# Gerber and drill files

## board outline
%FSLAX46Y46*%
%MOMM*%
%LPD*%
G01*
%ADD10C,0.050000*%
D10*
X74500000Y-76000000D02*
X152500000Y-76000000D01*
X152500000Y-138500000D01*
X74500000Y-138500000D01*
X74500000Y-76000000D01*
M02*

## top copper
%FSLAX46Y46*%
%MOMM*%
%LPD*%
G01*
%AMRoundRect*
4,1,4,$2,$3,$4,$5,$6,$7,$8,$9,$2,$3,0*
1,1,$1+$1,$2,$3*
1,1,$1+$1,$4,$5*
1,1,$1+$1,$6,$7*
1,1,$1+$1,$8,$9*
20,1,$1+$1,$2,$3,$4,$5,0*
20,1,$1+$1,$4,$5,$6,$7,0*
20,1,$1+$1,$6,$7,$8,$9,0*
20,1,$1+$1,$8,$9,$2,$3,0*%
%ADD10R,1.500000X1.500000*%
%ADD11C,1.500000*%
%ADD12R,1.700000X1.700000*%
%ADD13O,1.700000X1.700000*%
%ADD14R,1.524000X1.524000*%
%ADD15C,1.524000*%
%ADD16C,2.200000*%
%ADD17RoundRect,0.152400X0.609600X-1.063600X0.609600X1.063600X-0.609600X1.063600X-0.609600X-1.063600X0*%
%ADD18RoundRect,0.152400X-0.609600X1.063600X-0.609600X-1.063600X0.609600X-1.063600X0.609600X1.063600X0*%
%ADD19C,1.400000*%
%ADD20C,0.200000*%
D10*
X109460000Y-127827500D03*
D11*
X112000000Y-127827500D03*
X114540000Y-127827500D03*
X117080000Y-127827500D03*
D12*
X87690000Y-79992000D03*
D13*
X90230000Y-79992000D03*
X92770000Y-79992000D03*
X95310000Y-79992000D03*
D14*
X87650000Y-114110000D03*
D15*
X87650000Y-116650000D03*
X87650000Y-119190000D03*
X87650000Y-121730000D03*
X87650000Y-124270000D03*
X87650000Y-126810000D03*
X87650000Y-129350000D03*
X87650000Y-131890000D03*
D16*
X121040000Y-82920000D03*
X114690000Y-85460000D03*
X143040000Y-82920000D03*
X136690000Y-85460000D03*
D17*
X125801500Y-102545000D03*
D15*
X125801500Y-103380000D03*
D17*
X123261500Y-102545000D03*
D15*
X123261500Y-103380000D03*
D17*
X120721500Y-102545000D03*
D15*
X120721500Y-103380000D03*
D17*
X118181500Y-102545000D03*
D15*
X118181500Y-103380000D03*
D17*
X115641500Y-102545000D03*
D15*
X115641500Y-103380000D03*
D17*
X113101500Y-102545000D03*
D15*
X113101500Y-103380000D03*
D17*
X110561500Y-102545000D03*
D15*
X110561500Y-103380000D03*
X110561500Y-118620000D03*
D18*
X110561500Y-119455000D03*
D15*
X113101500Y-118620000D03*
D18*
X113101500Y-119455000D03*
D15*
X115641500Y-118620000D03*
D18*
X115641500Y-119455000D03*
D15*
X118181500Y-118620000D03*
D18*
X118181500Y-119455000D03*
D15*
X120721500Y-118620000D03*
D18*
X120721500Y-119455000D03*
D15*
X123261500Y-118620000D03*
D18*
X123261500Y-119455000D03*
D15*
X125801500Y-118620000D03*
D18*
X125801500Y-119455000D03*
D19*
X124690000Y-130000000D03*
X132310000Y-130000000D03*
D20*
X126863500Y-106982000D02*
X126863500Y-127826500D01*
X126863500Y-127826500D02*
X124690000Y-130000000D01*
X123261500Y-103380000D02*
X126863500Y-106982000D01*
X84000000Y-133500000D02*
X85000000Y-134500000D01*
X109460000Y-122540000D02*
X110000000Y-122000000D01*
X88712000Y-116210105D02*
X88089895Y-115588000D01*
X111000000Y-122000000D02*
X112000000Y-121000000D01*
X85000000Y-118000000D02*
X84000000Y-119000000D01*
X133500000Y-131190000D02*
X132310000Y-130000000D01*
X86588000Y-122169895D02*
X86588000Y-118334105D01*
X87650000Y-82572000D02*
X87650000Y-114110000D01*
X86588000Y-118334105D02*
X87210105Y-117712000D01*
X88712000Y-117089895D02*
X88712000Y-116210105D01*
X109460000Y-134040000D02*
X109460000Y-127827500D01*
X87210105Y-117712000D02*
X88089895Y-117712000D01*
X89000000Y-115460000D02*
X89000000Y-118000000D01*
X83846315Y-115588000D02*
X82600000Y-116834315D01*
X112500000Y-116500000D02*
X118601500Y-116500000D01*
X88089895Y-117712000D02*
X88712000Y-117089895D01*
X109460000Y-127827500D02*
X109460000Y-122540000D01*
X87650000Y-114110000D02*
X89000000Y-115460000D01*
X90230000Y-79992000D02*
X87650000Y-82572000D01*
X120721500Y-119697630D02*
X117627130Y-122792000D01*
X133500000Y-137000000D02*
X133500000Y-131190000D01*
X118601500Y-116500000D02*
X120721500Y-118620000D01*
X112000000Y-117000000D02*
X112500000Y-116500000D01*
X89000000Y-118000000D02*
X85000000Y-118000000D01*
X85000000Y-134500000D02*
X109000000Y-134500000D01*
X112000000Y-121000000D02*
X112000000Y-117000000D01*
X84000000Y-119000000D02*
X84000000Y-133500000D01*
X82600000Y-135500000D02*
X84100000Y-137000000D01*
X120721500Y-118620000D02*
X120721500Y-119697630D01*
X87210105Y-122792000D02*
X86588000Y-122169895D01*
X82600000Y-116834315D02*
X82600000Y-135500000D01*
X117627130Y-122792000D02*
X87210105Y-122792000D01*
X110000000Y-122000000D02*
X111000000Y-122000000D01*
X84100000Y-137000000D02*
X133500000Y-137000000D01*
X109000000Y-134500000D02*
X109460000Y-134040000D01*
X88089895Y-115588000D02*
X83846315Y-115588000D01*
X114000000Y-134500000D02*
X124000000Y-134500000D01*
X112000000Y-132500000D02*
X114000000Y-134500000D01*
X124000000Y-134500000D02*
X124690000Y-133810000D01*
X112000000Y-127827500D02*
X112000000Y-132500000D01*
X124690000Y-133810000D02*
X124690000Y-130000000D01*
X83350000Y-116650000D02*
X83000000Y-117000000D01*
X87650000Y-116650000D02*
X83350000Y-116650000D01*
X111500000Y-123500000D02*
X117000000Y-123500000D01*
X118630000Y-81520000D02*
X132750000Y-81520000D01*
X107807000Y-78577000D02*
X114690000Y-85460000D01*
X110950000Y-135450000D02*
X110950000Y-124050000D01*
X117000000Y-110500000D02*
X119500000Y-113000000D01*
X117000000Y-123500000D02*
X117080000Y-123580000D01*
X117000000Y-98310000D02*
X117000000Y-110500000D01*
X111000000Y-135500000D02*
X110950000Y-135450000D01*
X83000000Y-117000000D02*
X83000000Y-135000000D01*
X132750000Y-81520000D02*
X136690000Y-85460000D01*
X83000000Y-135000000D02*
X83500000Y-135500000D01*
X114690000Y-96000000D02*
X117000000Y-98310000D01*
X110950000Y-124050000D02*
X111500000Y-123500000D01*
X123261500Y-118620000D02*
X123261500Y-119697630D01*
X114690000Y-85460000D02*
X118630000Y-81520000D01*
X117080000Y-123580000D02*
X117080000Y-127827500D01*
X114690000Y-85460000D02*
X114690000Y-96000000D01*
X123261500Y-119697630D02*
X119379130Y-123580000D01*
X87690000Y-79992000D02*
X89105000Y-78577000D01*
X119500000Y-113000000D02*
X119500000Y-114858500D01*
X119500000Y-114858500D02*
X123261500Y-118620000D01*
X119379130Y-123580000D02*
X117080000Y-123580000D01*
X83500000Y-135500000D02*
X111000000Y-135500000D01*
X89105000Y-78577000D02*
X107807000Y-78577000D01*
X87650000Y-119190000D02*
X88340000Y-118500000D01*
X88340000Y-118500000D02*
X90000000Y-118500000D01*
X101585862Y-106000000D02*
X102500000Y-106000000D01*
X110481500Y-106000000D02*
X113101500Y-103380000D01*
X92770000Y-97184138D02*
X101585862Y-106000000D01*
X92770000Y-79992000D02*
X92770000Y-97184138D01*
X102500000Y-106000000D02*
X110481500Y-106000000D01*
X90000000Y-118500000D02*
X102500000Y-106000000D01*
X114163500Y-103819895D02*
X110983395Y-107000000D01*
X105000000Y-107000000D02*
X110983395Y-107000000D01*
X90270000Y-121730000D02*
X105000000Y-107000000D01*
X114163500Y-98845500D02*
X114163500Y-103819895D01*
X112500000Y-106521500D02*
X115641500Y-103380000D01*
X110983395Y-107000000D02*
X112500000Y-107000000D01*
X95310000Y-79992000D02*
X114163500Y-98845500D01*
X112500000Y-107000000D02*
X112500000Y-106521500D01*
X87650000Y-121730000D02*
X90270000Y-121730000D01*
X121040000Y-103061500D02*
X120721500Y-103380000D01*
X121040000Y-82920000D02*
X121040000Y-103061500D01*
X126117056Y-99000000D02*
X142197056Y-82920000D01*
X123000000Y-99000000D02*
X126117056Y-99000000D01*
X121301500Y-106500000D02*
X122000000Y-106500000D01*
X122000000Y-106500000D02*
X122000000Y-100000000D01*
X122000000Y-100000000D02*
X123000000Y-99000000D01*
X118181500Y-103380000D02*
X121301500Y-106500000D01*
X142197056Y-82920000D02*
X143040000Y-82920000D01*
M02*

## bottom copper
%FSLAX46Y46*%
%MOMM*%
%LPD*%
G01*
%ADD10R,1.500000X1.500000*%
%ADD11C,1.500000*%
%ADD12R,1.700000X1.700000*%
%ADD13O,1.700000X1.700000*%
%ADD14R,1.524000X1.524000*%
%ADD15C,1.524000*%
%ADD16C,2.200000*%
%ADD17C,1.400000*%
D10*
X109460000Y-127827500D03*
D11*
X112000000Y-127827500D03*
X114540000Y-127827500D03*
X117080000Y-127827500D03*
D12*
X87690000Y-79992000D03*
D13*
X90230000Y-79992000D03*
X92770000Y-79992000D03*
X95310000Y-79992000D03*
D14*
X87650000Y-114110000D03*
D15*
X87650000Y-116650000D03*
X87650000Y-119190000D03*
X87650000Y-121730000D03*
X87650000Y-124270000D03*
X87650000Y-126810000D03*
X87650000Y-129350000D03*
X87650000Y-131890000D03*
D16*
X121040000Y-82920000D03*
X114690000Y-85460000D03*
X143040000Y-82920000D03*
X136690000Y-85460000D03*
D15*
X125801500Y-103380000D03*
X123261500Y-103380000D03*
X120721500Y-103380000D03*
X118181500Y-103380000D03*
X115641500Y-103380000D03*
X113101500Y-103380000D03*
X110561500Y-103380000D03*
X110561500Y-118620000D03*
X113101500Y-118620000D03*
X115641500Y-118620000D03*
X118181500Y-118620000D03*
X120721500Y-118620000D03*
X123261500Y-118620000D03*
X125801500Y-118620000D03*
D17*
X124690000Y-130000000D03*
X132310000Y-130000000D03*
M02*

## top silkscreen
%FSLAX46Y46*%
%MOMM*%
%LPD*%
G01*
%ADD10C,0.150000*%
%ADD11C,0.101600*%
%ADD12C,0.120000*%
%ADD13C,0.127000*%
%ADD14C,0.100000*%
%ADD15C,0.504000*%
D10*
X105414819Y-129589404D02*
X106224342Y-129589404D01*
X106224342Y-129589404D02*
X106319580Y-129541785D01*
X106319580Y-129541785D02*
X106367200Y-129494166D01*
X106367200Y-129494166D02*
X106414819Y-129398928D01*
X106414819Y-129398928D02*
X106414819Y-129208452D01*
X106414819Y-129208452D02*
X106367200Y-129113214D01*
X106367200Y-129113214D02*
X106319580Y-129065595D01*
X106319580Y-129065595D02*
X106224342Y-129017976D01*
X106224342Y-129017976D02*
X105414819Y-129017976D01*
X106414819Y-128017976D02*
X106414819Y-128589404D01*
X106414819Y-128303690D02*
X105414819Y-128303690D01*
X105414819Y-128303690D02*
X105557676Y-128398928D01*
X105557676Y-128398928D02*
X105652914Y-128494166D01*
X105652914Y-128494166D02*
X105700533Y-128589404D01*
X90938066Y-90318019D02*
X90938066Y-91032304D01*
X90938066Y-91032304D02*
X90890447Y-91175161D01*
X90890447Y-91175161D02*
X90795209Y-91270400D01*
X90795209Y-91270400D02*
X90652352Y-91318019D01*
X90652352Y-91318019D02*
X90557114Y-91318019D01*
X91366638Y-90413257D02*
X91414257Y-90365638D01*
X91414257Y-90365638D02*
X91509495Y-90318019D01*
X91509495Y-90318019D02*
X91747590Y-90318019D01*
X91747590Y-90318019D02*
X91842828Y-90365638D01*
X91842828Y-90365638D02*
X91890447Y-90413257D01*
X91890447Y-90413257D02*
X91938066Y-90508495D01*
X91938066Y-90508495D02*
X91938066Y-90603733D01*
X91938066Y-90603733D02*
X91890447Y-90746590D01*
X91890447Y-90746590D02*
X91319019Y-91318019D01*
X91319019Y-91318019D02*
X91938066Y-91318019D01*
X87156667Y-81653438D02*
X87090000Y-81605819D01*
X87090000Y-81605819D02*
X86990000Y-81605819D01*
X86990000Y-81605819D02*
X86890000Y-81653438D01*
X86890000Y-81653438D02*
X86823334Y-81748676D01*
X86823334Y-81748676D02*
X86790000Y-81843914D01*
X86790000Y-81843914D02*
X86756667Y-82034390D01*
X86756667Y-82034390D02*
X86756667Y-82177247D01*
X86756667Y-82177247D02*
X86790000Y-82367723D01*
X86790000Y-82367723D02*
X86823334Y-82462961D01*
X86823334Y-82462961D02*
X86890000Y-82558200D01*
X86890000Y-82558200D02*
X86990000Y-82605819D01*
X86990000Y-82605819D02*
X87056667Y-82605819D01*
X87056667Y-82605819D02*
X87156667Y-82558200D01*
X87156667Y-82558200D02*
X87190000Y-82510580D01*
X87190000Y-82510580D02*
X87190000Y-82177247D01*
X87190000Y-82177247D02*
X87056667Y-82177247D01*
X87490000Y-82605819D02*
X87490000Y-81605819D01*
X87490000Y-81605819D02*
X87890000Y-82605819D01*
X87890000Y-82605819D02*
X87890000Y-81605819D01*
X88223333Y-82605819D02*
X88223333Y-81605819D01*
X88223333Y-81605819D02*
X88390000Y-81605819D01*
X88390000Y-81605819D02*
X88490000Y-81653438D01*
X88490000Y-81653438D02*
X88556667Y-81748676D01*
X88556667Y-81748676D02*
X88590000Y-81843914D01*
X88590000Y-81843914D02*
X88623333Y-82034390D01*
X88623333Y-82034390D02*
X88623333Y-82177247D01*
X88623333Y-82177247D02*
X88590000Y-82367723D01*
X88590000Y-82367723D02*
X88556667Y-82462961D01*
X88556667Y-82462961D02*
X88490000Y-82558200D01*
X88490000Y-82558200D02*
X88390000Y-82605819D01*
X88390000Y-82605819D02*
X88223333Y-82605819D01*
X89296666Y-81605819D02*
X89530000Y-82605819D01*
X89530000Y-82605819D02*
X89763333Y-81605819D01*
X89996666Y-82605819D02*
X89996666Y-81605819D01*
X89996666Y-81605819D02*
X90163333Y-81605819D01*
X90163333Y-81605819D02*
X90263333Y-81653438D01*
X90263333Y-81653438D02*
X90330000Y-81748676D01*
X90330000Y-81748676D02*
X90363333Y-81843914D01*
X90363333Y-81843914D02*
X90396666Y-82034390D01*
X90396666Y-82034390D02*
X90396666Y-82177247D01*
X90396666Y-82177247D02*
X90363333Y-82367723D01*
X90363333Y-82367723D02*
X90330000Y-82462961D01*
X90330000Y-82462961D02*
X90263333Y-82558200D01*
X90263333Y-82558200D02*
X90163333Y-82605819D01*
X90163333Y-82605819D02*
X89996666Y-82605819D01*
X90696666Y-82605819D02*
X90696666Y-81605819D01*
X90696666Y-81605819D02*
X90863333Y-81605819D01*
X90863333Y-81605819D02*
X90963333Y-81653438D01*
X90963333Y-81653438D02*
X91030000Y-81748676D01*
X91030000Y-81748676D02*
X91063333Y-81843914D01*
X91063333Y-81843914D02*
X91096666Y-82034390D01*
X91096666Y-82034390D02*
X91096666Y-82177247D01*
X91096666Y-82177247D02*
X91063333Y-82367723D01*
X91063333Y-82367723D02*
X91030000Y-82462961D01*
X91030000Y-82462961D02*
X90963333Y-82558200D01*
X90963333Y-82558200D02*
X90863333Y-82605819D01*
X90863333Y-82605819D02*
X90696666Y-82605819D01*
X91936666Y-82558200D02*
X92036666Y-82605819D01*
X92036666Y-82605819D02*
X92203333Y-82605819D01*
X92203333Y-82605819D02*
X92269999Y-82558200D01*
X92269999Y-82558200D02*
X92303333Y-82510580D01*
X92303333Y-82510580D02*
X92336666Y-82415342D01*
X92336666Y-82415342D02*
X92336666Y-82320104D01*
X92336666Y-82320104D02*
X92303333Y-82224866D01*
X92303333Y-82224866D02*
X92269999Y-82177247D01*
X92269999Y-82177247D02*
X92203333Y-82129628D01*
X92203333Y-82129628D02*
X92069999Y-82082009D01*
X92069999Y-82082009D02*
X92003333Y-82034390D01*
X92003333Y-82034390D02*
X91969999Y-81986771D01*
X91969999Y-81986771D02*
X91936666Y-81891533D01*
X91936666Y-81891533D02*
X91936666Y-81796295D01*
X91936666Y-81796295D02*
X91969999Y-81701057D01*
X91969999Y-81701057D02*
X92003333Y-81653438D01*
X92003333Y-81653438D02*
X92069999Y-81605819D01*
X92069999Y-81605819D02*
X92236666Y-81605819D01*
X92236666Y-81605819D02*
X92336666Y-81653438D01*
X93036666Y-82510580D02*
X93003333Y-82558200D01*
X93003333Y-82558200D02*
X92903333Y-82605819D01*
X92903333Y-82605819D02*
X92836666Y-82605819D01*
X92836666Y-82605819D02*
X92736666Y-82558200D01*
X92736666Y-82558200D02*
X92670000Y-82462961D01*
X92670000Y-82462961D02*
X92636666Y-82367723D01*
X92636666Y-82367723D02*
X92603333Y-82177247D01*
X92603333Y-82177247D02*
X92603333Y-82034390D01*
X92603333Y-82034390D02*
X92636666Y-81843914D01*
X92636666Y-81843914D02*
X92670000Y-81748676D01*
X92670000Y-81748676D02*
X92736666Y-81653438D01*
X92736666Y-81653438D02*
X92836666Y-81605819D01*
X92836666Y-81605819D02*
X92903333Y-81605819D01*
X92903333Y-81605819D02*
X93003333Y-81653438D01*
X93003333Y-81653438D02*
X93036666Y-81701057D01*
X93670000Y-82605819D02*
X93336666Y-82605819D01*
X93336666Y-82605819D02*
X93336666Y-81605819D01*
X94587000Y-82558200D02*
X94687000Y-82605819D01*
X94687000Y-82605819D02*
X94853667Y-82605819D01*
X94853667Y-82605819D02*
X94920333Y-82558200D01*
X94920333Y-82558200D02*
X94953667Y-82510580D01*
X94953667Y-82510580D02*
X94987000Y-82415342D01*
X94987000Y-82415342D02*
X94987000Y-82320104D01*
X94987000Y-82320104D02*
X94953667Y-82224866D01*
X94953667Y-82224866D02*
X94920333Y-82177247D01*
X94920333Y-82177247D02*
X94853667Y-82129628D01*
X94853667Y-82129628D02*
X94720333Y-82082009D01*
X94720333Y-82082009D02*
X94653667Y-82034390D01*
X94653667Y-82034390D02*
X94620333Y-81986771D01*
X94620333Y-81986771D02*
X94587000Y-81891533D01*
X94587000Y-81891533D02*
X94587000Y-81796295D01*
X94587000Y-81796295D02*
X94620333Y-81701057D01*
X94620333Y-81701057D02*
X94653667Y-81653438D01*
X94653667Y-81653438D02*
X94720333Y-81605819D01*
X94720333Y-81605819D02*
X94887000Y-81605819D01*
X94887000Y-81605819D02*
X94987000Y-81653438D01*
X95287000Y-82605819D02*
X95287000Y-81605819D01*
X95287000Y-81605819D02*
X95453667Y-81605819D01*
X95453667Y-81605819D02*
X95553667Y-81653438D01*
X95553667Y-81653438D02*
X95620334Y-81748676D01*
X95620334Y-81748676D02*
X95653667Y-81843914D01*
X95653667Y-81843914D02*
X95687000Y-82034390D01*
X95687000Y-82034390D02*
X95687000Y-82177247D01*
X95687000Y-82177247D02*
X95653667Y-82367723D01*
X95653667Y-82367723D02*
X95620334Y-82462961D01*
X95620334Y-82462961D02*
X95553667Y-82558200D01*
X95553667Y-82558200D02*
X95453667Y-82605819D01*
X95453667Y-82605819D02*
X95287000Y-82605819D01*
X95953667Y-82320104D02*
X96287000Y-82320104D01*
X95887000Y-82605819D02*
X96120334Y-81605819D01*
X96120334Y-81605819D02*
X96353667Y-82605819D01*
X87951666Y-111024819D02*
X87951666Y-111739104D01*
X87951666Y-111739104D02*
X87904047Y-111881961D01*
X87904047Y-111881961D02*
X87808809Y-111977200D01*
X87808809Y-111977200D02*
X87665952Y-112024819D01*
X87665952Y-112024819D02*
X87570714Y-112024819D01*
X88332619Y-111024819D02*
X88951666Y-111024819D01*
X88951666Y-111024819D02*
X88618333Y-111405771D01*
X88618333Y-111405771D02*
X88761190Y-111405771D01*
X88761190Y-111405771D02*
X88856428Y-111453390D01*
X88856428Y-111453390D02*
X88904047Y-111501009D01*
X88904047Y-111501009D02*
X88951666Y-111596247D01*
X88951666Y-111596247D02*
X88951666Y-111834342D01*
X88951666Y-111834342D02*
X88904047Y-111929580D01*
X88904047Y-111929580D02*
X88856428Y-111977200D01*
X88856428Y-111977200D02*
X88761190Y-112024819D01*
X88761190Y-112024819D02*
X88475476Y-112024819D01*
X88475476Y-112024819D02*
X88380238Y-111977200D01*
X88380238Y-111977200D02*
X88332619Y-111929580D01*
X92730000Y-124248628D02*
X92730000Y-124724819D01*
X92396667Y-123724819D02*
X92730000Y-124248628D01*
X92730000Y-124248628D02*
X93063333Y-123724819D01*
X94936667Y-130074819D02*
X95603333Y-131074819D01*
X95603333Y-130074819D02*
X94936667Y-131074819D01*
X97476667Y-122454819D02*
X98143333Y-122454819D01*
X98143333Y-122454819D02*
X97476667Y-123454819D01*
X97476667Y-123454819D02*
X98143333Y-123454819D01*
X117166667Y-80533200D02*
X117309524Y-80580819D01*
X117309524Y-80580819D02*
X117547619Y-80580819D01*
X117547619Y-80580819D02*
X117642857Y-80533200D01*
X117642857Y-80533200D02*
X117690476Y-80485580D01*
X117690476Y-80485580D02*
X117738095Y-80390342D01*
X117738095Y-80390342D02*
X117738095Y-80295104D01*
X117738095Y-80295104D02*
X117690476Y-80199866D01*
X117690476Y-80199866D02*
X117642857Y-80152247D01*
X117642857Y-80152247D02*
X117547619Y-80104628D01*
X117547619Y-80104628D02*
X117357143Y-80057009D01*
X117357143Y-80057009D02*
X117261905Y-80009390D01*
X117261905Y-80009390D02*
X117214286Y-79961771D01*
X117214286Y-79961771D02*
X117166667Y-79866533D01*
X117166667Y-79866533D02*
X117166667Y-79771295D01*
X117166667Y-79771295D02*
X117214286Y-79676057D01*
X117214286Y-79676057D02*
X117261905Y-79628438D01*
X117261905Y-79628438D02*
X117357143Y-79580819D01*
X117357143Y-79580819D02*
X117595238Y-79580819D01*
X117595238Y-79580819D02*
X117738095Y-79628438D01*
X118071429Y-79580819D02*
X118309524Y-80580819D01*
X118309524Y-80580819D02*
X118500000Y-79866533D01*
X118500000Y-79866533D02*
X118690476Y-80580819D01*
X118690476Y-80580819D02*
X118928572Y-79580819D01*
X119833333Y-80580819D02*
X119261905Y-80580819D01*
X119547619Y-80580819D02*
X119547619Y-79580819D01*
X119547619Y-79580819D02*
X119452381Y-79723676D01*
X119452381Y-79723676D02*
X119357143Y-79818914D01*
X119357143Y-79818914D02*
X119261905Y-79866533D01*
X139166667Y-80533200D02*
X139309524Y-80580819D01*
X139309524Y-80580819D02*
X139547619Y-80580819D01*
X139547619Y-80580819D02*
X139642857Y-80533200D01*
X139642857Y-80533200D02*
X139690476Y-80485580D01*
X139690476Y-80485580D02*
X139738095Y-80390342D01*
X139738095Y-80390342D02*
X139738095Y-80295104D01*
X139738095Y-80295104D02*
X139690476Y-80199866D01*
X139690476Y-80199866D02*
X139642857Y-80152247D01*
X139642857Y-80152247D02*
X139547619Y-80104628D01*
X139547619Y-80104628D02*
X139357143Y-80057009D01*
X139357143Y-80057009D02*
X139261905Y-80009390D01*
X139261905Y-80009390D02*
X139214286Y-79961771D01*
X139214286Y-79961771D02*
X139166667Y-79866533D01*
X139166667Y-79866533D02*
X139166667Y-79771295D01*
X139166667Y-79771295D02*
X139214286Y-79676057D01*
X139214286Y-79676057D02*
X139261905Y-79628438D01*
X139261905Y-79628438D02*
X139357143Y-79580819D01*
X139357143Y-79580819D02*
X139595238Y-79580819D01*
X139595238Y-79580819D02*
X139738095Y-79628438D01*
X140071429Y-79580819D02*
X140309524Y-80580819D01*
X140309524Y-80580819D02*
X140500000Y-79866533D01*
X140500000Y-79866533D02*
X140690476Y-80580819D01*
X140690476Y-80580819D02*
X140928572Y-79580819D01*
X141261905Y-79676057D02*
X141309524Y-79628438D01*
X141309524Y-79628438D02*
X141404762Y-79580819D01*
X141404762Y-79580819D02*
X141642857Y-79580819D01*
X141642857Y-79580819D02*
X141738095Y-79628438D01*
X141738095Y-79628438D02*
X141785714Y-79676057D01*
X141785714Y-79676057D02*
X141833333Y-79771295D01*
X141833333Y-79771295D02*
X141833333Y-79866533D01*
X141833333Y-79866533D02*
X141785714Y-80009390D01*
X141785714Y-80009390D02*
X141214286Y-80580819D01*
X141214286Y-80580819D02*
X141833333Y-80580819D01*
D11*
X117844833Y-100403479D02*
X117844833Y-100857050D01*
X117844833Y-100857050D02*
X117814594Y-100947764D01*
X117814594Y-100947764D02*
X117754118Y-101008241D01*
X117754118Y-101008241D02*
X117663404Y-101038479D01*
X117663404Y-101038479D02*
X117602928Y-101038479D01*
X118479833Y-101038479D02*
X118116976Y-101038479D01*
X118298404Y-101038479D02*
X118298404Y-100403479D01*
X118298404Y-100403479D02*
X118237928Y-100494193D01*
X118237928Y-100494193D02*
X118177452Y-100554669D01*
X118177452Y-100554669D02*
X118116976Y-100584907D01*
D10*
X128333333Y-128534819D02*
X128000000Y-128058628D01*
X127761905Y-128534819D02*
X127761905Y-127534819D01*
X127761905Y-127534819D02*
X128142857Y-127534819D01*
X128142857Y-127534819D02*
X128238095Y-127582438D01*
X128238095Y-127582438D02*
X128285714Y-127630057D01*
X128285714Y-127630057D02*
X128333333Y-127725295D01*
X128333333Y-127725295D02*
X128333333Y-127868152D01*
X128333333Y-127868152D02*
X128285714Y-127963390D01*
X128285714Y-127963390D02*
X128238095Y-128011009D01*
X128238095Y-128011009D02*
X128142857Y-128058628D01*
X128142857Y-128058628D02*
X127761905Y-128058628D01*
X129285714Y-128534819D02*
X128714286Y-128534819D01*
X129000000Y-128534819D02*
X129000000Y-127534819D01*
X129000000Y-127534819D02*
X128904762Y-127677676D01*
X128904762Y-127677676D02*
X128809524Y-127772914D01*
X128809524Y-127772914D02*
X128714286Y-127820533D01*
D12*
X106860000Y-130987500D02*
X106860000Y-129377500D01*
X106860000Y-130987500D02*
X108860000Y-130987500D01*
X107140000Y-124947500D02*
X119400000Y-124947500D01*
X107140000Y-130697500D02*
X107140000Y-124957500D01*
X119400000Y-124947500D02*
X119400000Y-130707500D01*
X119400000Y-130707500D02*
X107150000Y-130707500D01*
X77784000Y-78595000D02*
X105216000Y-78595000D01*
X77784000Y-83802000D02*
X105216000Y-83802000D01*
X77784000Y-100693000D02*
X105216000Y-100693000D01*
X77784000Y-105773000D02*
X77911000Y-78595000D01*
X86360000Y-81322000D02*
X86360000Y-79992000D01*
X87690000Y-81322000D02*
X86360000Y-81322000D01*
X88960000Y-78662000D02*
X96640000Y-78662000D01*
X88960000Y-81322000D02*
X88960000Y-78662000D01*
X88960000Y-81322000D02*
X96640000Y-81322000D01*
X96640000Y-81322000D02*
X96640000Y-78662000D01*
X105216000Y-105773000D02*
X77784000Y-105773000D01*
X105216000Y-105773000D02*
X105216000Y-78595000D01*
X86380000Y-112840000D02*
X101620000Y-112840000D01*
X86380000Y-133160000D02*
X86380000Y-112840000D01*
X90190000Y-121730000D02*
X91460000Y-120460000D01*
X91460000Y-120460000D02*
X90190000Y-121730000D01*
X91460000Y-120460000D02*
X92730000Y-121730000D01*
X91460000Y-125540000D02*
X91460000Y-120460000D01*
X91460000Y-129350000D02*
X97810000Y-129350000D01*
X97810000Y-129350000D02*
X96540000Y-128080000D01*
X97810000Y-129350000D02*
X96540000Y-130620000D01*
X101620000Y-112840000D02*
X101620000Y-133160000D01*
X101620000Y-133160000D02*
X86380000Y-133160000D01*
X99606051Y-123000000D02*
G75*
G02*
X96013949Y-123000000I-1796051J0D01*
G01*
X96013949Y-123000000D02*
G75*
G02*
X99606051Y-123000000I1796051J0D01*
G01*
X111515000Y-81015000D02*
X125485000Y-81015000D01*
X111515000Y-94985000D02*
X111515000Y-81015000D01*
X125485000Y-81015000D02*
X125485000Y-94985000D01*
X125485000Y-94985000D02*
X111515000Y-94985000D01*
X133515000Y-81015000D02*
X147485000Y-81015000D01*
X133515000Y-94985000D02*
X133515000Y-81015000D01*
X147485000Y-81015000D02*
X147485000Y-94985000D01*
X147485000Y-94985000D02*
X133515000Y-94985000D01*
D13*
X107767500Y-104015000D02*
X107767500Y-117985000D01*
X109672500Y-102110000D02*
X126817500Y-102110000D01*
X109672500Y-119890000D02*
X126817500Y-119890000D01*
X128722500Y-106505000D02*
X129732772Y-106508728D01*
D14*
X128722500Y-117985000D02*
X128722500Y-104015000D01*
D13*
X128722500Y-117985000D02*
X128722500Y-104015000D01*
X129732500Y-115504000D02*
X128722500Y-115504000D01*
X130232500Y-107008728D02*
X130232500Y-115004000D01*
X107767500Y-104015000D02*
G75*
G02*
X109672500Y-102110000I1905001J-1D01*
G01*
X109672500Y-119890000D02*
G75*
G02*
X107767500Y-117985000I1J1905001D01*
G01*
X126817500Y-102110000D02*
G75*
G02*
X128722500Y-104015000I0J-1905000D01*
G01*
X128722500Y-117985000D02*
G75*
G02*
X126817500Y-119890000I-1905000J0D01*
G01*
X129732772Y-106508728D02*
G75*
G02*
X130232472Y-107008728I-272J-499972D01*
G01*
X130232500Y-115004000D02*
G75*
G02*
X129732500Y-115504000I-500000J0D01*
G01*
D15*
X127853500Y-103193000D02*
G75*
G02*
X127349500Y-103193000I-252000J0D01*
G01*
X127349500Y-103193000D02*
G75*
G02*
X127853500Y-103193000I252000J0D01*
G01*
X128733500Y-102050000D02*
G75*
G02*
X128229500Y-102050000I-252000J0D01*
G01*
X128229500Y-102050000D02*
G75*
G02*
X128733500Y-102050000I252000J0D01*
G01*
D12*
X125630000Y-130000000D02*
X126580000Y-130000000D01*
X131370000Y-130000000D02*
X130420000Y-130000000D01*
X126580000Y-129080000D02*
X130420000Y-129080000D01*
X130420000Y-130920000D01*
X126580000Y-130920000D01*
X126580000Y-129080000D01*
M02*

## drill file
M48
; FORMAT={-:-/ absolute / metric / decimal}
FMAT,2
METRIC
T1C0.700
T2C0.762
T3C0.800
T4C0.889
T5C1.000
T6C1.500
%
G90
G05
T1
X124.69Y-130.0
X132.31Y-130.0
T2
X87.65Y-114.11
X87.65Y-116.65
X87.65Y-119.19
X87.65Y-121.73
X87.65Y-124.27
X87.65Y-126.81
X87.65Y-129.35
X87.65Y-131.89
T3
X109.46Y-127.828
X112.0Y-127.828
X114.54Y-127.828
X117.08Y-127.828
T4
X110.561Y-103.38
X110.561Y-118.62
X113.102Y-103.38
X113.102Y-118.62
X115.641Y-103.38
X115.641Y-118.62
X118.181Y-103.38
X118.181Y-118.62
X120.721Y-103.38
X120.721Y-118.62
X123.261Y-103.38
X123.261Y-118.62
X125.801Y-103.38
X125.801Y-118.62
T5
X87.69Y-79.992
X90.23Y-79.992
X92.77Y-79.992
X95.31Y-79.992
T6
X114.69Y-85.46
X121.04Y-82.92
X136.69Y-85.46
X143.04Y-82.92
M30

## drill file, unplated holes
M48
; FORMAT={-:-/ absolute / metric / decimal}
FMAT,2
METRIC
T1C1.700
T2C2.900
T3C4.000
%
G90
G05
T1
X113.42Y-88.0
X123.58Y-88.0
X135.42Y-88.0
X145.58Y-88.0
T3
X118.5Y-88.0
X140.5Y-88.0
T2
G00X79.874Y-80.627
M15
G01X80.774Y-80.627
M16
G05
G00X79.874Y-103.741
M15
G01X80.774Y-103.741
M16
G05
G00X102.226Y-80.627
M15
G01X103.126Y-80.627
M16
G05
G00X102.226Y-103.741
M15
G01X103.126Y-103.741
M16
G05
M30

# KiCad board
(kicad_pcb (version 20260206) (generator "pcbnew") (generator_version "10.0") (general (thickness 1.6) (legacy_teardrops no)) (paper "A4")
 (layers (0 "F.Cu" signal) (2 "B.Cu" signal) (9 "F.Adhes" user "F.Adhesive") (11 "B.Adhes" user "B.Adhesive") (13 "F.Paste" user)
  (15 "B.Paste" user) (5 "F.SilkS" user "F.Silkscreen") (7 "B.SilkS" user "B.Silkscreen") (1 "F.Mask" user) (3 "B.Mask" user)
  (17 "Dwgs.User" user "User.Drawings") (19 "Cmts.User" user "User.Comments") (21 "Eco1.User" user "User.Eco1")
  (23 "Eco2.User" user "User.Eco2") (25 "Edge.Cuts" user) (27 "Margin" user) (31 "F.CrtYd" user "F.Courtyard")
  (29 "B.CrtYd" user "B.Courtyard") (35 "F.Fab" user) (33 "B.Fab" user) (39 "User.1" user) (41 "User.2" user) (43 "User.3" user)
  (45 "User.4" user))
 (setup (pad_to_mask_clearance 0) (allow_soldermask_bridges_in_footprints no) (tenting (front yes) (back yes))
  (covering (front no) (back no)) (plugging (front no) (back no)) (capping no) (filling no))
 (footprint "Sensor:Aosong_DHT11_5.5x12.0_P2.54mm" (layer "F.Cu") (at 109.46 127.8275 90)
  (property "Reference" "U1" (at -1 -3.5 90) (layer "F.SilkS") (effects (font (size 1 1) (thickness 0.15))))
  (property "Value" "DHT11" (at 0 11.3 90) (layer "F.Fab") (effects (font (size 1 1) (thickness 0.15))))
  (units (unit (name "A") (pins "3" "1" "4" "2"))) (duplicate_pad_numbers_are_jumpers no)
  (fp_line (start -3.16 -2.6) (end -1.55 -2.6) (stroke (width 0.12) (type solid)) (layer "F.SilkS"))
  (fp_line (start -3.16 -2.6) (end -3.16 -0.6) (stroke (width 0.12) (type solid)) (layer "F.SilkS"))
  (fp_line (start 2.88 -2.32) (end 2.88 9.94) (stroke (width 0.12) (type solid)) (layer "F.SilkS"))
  (fp_line (start -2.87 -2.32) (end 2.87 -2.32) (stroke (width 0.12) (type solid)) (layer "F.SilkS"))
  (fp_line (start 2.88 9.94) (end -2.88 9.94) (stroke (width 0.12) (type solid)) (layer "F.SilkS"))
  (fp_line (start -2.88 9.94) (end -2.88 -2.31) (stroke (width 0.12) (type solid)) (layer "F.SilkS"))
  (pad "1" thru_hole rect (at 0 0 90) (size 1.5 1.5) (drill 0.8) (layers "*.Cu" "*.Mask") (remove_unused_layers no) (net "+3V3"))
  (pad "2" thru_hole circle (at 0 2.54 90) (size 1.5 1.5) (drill 0.8) (layers "*.Cu" "*.Mask") (remove_unused_layers no) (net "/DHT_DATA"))
  (pad "3" thru_hole circle (at 0 5.08 90) (size 1.5 1.5) (drill 0.8) (layers "*.Cu" "*.Mask") (remove_unused_layers no)
   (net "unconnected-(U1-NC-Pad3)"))
  (pad "4" thru_hole circle (at 0 7.62 90) (size 1.5 1.5) (drill 0.8) (layers "*.Cu" "*.Mask") (remove_unused_layers no) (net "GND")))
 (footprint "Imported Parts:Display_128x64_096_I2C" (layer "F.Cu") (at 91.5 79.992)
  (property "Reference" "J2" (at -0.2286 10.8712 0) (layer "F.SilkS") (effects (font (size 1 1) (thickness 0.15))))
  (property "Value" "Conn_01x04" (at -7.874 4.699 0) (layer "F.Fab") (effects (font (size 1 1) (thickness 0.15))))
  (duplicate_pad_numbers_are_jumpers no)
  (fp_line (start -13.716 -1.397) (end 13.716 -1.397) (stroke (width 0.12) (type solid)) (layer "F.SilkS"))
  (fp_line (start -13.716 3.81) (end 13.716 3.81) (stroke (width 0.12) (type solid)) (layer "F.SilkS"))
  (fp_line (start -13.716 20.701) (end 13.716 20.701) (stroke (width 0.12) (type solid)) (layer "F.SilkS"))
  (fp_line (start -13.716 25.781) (end -13.589 -1.397) (stroke (width 0.12) (type solid)) (layer "F.SilkS"))
  (fp_line (start -5.14 1.33) (end -5.14 0) (stroke (width 0.12) (type solid)) (layer "F.SilkS"))
  (fp_line (start -3.81 1.33) (end -5.14 1.33) (stroke (width 0.12) (type solid)) (layer "F.SilkS"))
  (fp_line (start -2.54 -1.33) (end 5.14 -1.33) (stroke (width 0.12) (type solid)) (layer "F.SilkS"))
  (fp_line (start -2.54 1.33) (end -2.54 -1.33) (stroke (width 0.12) (type solid)) (layer "F.SilkS"))
  (fp_line (start -2.54 1.33) (end 5.14 1.33) (stroke (width 0.12) (type solid)) (layer "F.SilkS"))
  (fp_line (start 5.14 1.33) (end 5.14 -1.33) (stroke (width 0.12) (type solid)) (layer "F.SilkS"))
  (fp_line (start 13.716 25.781) (end -13.716 25.781) (stroke (width 0.12) (type solid)) (layer "F.SilkS"))
  (fp_line (start 13.716 25.781) (end 13.716 -1.397) (stroke (width 0.12) (type solid)) (layer "F.SilkS"))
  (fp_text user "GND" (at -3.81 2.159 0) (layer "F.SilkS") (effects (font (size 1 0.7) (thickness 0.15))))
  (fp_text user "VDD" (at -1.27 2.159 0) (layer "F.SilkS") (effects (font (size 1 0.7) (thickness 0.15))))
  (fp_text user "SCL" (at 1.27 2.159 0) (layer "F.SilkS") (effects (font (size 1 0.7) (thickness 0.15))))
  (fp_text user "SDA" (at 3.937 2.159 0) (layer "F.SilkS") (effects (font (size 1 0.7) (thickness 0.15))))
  (pad "" np_thru_hole oval (at -11.176 0.635) (size 3.8 2.9) (drill oval 3.8 2.9) (layers "*.Cu" "*.Mask"))
  (pad "" np_thru_hole oval (at -11.176 23.749) (size 3.8 2.9) (drill oval 3.8 2.9) (layers "*.Cu" "*.Mask"))
  (pad "" np_thru_hole oval (at 11.176 0.635) (size 3.8 2.9) (drill oval 3.8 2.9) (layers "*.Cu" "*.Mask"))
  (pad "" np_thru_hole oval (at 11.176 23.749) (size 3.8 2.9) (drill oval 3.8 2.9) (layers "*.Cu" "*.Mask"))
  (pad "1" thru_hole rect (at -3.81 0 90) (size 1.7 1.7) (drill 1) (layers "*.Cu" "*.Mask") (remove_unused_layers no) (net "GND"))
  (pad "2" thru_hole oval (at -1.27 0 90) (size 1.7 1.7) (drill 1) (layers "*.Cu" "*.Mask") (remove_unused_layers no) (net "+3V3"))
  (pad "3" thru_hole oval (at 1.27 0 90) (size 1.7 1.7) (drill 1) (layers "*.Cu" "*.Mask") (remove_unused_layers no) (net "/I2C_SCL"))
  (pad "4" thru_hole oval (at 3.81 0 90) (size 1.7 1.7) (drill 1) (layers "*.Cu" "*.Mask") (remove_unused_layers no) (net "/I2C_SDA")))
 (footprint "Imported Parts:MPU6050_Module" (layer "F.Cu") (at 87.65 114.11)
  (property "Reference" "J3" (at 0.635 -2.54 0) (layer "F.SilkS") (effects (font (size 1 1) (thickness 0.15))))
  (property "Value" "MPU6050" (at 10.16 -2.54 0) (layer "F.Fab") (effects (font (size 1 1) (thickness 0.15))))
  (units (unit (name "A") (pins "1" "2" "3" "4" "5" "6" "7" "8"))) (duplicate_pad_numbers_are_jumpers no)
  (fp_line (start -1.27 -1.27) (end 13.97 -1.27) (stroke (width 0.12) (type solid)) (layer "F.SilkS"))
  (fp_line (start -1.27 19.05) (end -1.27 -1.27) (stroke (width 0.12) (type solid)) (layer "F.SilkS"))
  (fp_line (start 2.54 7.62) (end 3.81 6.35) (stroke (width 0.12) (type solid)) (layer "F.SilkS"))
  (fp_line (start 3.81 6.35) (end 2.54 7.62) (stroke (width 0.12) (type solid)) (layer "F.SilkS"))
  (fp_line (start 3.81 6.35) (end 5.08 7.62) (stroke (width 0.12) (type solid)) (layer "F.SilkS"))
  (fp_line (start 3.81 11.43) (end 3.81 6.35) (stroke (width 0.12) (type solid)) (layer "F.SilkS"))
  (fp_line (start 3.81 15.24) (end 10.16 15.24) (stroke (width 0.12) (type solid)) (layer "F.SilkS"))
  (fp_line (start 10.16 15.24) (end 8.89 13.97) (stroke (width 0.12) (type solid)) (layer "F.SilkS"))
  (fp_line (start 10.16 15.24) (end 8.89 16.51) (stroke (width 0.12) (type solid)) (layer "F.SilkS"))
  (fp_line (start 13.97 -1.27) (end 13.97 19.05) (stroke (width 0.12) (type solid)) (layer "F.SilkS"))
  (fp_line (start 13.97 19.05) (end -1.27 19.05) (stroke (width 0.12) (type solid)) (layer "F.SilkS"))
  (fp_circle (center 10.16 8.89) (end 8.89 7.62) (stroke (width 0.12) (type solid)) (fill no) (layer "F.SilkS"))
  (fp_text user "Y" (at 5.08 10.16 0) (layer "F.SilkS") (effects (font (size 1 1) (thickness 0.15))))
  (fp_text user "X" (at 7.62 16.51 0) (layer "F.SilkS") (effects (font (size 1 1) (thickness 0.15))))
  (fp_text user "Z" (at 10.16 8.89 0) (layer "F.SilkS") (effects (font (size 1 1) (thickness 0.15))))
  (pad "1" thru_hole rect (at 0 0) (size 1.524 1.524) (drill 0.762) (layers "*.Cu" "*.Mask") (remove_unused_layers no) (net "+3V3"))
  (pad "2" thru_hole circle (at 0 2.54) (size 1.524 1.524) (drill 0.762) (layers "*.Cu" "*.Mask") (remove_unused_layers no) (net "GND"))
  (pad "3" thru_hole circle (at 0 5.08) (size 1.524 1.524) (drill 0.762) (layers "*.Cu" "*.Mask") (remove_unused_layers no) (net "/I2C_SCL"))
  (pad "4" thru_hole circle (at 0 7.62) (size 1.524 1.524) (drill 0.762) (layers "*.Cu" "*.Mask") (remove_unused_layers no) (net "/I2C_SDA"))
  (pad "5" thru_hole circle (at 0 10.16) (size 1.524 1.524) (drill 0.762) (layers "*.Cu" "*.Mask") (remove_unused_layers no)
   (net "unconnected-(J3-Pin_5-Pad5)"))
  (pad "6" thru_hole circle (at 0 12.7) (size 1.524 1.524) (drill 0.762) (layers "*.Cu" "*.Mask") (remove_unused_layers no)
   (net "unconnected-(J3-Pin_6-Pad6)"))
  (pad "7" thru_hole circle (at 0 15.24) (size 1.524 1.524) (drill 0.762) (layers "*.Cu" "*.Mask") (remove_unused_layers no)
   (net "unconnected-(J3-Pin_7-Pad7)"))
  (pad "8" thru_hole circle (at 0 17.78) (size 1.524 1.524) (drill 0.762) (layers "*.Cu" "*.Mask") (remove_unused_layers no)
   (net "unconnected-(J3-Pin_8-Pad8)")))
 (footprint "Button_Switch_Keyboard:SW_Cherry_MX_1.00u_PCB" (layer "F.Cu") (at 121.04 82.92)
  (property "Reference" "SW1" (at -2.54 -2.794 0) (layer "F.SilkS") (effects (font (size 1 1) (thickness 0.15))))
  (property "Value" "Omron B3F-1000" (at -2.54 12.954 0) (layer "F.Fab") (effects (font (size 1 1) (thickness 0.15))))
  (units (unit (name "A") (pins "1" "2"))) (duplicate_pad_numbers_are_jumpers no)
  (fp_line (start -9.525 -1.905) (end 4.445 -1.905) (stroke (width 0.12) (type solid)) (layer "F.SilkS"))
  (fp_line (start -9.525 12.065) (end -9.525 -1.905) (stroke (width 0.12) (type solid)) (layer "F.SilkS"))
  (fp_line (start 4.445 -1.905) (end 4.445 12.065) (stroke (width 0.12) (type solid)) (layer "F.SilkS"))
  (fp_line (start 4.445 12.065) (end -9.525 12.065) (stroke (width 0.12) (type solid)) (layer "F.SilkS"))
  (pad "" np_thru_hole circle (at -7.62 5.08) (size 1.7 1.7) (drill 1.7) (layers "*.Cu" "*.Mask"))
  (pad "" np_thru_hole circle (at -2.54 5.08) (size 4 4) (drill 4) (layers "*.Cu" "*.Mask"))
  (pad "" np_thru_hole circle (at 2.54 5.08) (size 1.7 1.7) (drill 1.7) (layers "*.Cu" "*.Mask"))
  (pad "1" thru_hole circle (at 0 0) (size 2.2 2.2) (drill 1.5) (layers "*.Cu" "*.Mask") (remove_unused_layers no) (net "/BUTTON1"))
  (pad "2" thru_hole circle (at -6.35 2.54) (size 2.2 2.2) (drill 1.5) (layers "*.Cu" "*.Mask") (remove_unused_layers no) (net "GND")))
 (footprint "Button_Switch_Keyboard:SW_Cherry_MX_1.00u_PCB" (layer "F.Cu") (at 143.04 82.92)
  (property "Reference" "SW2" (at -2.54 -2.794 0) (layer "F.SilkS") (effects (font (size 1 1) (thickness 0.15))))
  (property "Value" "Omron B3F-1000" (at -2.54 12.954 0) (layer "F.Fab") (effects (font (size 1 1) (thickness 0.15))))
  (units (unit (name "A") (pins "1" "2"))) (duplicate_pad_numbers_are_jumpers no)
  (fp_line (start -9.525 -1.905) (end 4.445 -1.905) (stroke (width 0.12) (type solid)) (layer "F.SilkS"))
  (fp_line (start -9.525 12.065) (end -9.525 -1.905) (stroke (width 0.12) (type solid)) (layer "F.SilkS"))
  (fp_line (start 4.445 -1.905) (end 4.445 12.065) (stroke (width 0.12) (type solid)) (layer "F.SilkS"))
  (fp_line (start 4.445 12.065) (end -9.525 12.065) (stroke (width 0.12) (type solid)) (layer "F.SilkS"))
  (pad "" np_thru_hole circle (at -7.62 5.08) (size 1.7 1.7) (drill 1.7) (layers "*.Cu" "*.Mask"))
  (pad "" np_thru_hole circle (at -2.54 5.08) (size 4 4) (drill 4) (layers "*.Cu" "*.Mask"))
  (pad "" np_thru_hole circle (at 2.54 5.08) (size 1.7 1.7) (drill 1.7) (layers "*.Cu" "*.Mask"))
  (pad "1" thru_hole circle (at 0 0) (size 2.2 2.2) (drill 1.5) (layers "*.Cu" "*.Mask") (remove_unused_layers no) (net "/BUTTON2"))
  (pad "2" thru_hole circle (at -6.35 2.54) (size 2.2 2.2) (drill 1.5) (layers "*.Cu" "*.Mask") (remove_unused_layers no) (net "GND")))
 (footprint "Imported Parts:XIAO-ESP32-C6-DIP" (layer "F.Cu") (at 118.1815 111)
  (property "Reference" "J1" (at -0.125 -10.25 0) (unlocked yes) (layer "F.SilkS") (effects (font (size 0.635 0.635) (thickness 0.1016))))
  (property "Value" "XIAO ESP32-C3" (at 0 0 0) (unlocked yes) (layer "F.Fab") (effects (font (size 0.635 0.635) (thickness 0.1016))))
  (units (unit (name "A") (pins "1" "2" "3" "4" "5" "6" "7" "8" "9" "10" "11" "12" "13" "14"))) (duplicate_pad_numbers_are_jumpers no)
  (fp_line (start -10.414 -6.985) (end -10.414 6.985) (stroke (width 0.127) (type solid)) (layer "F.SilkS"))
  (fp_line (start -8.509 -8.89) (end 8.636 -8.89) (stroke (width 0.127) (type solid)) (layer "F.SilkS"))
  (fp_line (start -8.509 8.89) (end 8.636 8.89) (stroke (width 0.127) (type solid)) (layer "F.SilkS"))
  (fp_line (start 10.541 -4.495) (end 11.551272 -4.491272) (stroke (width 0.127) (type solid)) (layer "F.SilkS"))
  (fp_line (start 10.541 6.985) (end 10.541 -6.985) (stroke (width 0.1) (type solid)) (layer "F.SilkS"))
  (fp_line (start 10.541 6.985) (end 10.541 -6.985) (stroke (width 0.127) (type solid)) (layer "F.SilkS"))
  (fp_line (start 11.551 4.504) (end 10.541 4.504) (stroke (width 0.127) (type solid)) (layer "F.SilkS"))
  (fp_line (start 12.051 -3.991272) (end 12.051 4.004) (stroke (width 0.127) (type solid)) (layer "F.SilkS"))
  (fp_arc (start -10.414 -6.985) (mid -9.856038 -8.332038) (end -8.509 -8.89) (stroke (width 0.127) (type solid)) (layer "F.SilkS"))
  (fp_arc (start -8.509 8.89) (mid -9.856038 8.332038) (end -10.414 6.985) (stroke (width 0.127) (type solid)) (layer "F.SilkS"))
  (fp_arc (start 8.636 -8.89) (mid 9.983038 -8.332038) (end 10.541 -6.985) (stroke (width 0.127) (type solid)) (layer "F.SilkS"))
  (fp_arc (start 10.541 6.985) (mid 9.983038 8.332038) (end 8.636 8.89) (stroke (width 0.127) (type solid)) (layer "F.SilkS"))
  (fp_arc (start 11.551272 -4.491272) (mid 11.904644 -4.344724) (end 12.051 -3.991272) (stroke (width 0.127) (type default))
   (layer "F.SilkS"))
  (fp_arc (start 12.051 4.004) (mid 11.904553 4.357553) (end 11.551 4.504) (stroke (width 0.127) (type default)) (layer "F.SilkS"))
  (fp_circle (center 9.42 -7.807) (end 9.674 -7.807) (stroke (width 0.5) (type solid)) (fill yes) (layer "F.SilkS"))
  (fp_circle (center 10.3 -8.95) (end 10.554 -8.95) (stroke (width 0.5) (type solid)) (fill yes) (layer "F.SilkS"))
  (pad "1" smd roundrect (at 7.62 -8.455 90) (size 2.432 1.524) (layers "F.Cu" "F.Mask") (roundrect_rratio 0.1)
   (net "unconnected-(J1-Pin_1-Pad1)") (thermal_bridge_angle 45))
  (pad "1" thru_hole circle (at 7.62 -7.62 90) (size 1.524 1.524) (drill 0.889) (layers "*.Cu" "*.Mask") (remove_unused_layers no)
   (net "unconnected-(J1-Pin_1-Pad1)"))
  (pad "2" smd roundrect (at 5.08 -8.455 90) (size 2.432 1.524) (layers "F.Cu" "F.Mask") (roundrect_rratio 0.1) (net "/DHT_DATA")
   (thermal_bridge_angle 45))
  (pad "2" thru_hole circle (at 5.08 -7.62 90) (size 1.524 1.524) (drill 0.889) (layers "*.Cu" "*.Mask") (remove_unused_layers no)
   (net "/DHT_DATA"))
  (pad "3" smd roundrect (at 2.54 -8.455 90) (size 2.432 1.524) (layers "F.Cu" "F.Mask") (roundrect_rratio 0.1) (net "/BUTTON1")
   (thermal_bridge_angle 45))
  (pad "3" thru_hole circle (at 2.54 -7.62 90) (size 1.524 1.524) (drill 0.889) (layers "*.Cu" "*.Mask") (remove_unused_layers no)
   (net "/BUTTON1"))
  (pad "4" smd roundrect (at 0 -8.455 90) (size 2.432 1.524) (layers "F.Cu" "F.Mask") (roundrect_rratio 0.1) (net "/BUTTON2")
   (thermal_bridge_angle 45))
  (pad "4" thru_hole circle (at 0 -7.62 90) (size 1.524 1.524) (drill 0.889) (layers "*.Cu" "*.Mask") (remove_unused_layers no)
   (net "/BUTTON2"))
  (pad "5" smd roundrect (at -2.54 -8.455 90) (size 2.432 1.524) (layers "F.Cu" "F.Mask") (roundrect_rratio 0.1) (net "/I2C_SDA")
   (thermal_bridge_angle 45))
  (pad "5" thru_hole circle (at -2.54 -7.62 90) (size 1.524 1.524) (drill 0.889) (layers "*.Cu" "*.Mask") (remove_unused_layers no)
   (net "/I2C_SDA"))
  (pad "6" smd roundrect (at -5.08 -8.455 90) (size 2.432 1.524) (layers "F.Cu" "F.Mask") (roundrect_rratio 0.1) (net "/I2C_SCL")
   (thermal_bridge_angle 45))
  (pad "6" thru_hole circle (at -5.08 -7.62 90) (size 1.524 1.524) (drill 0.889) (layers "*.Cu" "*.Mask") (remove_unused_layers no)
   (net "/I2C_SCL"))
  (pad "7" smd roundrect (at -7.62 -8.455 90) (size 2.432 1.524) (layers "F.Cu" "F.Mask") (roundrect_rratio 0.1)
   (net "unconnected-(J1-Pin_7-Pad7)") (thermal_bridge_angle 45))
  (pad "7" thru_hole circle (at -7.62 -7.62 90) (size 1.524 1.524) (drill 0.889) (layers "*.Cu" "*.Mask") (remove_unused_layers no)
   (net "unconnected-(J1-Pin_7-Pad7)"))
  (pad "8" thru_hole circle (at -7.62 7.62 270) (size 1.524 1.524) (drill 0.889) (layers "*.Cu" "*.Mask") (remove_unused_layers no)
   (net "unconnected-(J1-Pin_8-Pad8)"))
  (pad "8" smd roundrect (at -7.62 8.455 270) (size 2.432 1.524) (layers "F.Cu" "F.Mask") (roundrect_rratio 0.1)
   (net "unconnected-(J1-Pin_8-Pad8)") (thermal_bridge_angle 45))
  (pad "9" thru_hole circle (at -5.08 7.62 270) (size 1.524 1.524) (drill 0.889) (layers "*.Cu" "*.Mask") (remove_unused_layers no)
   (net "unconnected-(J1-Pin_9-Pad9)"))
  (pad "9" smd roundrect (at -5.08 8.455 270) (size 2.432 1.524) (layers "F.Cu" "F.Mask") (roundrect_rratio 0.1)
   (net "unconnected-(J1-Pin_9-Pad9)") (thermal_bridge_angle 45))
  (pad "10" thru_hole circle (at -2.54 7.62 270) (size 1.524 1.524) (drill 0.889) (layers "*.Cu" "*.Mask") (remove_unused_layers no)
   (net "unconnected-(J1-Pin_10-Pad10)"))
  (pad "10" smd roundrect (at -2.54 8.455 270) (size 2.432 1.524) (layers "F.Cu" "F.Mask") (roundrect_rratio 0.1)
   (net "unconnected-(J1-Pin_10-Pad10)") (thermal_bridge_angle 45))
  (pad "11" thru_hole circle (at 0 7.62 270) (size 1.524 1.524) (drill 0.889) (layers "*.Cu" "*.Mask") (remove_unused_layers no)
   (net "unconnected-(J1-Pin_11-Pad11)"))
  (pad "11" smd roundrect (at 0 8.455 270) (size 2.432 1.524) (layers "F.Cu" "F.Mask") (roundrect_rratio 0.1)
   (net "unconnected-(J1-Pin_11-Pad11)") (thermal_bridge_angle 45))
  (pad "12" thru_hole circle (at 2.54 7.62 270) (size 1.524 1.524) (drill 0.889) (layers "*.Cu" "*.Mask") (remove_unused_layers no)
   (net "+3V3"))
  (pad "12" smd roundrect (at 2.54 8.455 270) (size 2.432 1.524) (layers "F.Cu" "F.Mask") (roundrect_rratio 0.1) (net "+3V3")
   (thermal_bridge_angle 45))
  (pad "13" thru_hole circle (at 5.08 7.62 270) (size 1.524 1.524) (drill 0.889) (layers "*.Cu" "*.Mask") (remove_unused_layers no)
   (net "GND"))
  (pad "13" smd roundrect (at 5.08 8.455 270) (size 2.432 1.524) (layers "F.Cu" "F.Mask") (roundrect_rratio 0.1) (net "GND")
   (thermal_bridge_angle 45))
  (pad "14" thru_hole circle (at 7.62 7.62 270) (size 1.524 1.524) (drill 0.889) (layers "*.Cu" "*.Mask") (remove_unused_layers no)
   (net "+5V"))
  (pad "14" smd roundrect (at 7.62 8.455 270) (size 2.432 1.524) (layers "F.Cu" "F.Mask") (roundrect_rratio 0.1) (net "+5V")
   (thermal_bridge_angle 45)))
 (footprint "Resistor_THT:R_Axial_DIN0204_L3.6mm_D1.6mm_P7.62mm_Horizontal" (layer "F.Cu") (at 124.69 130)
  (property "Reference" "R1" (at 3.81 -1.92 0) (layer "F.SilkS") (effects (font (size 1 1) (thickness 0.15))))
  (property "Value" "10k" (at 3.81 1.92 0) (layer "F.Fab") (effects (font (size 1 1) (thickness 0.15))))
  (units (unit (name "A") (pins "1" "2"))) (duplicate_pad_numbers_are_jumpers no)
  (fp_line (start 0.94 0) (end 1.89 0) (stroke (width 0.12) (type solid)) (layer "F.SilkS"))
  (fp_line (start 6.68 0) (end 5.73 0) (stroke (width 0.12) (type solid)) (layer "F.SilkS"))
  (fp_rect (start 1.89 -0.92) (end 5.73 0.92) (stroke (width 0.12) (type solid)) (fill no) (layer "F.SilkS"))
  (pad "1" thru_hole circle (at 0 0) (size 1.4 1.4) (drill 0.7) (layers "*.Cu" "*.Mask") (remove_unused_layers no) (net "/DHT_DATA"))
  (pad "2" thru_hole circle (at 7.62 0) (size 1.4 1.4) (drill 0.7) (layers "*.Cu" "*.Mask") (remove_unused_layers no) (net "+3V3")))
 (gr_rect (start 74.5 76) (end 152.5 138.5) (stroke (width 0.05) (type default)) (fill no) (layer "Edge.Cuts"))
 (segment (start 84 133.5) (end 85 134.5) (width 0.2) (layer "F.Cu") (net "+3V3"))
 (segment (start 109.46 122.54) (end 110 122) (width 0.2) (layer "F.Cu") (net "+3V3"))
 (segment (start 88.712 116.210105) (end 88.089895 115.588) (width 0.2) (layer "F.Cu") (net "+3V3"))
 (segment (start 111 122) (end 112 121) (width 0.2) (layer "F.Cu") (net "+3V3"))
 (segment (start 85 118) (end 84 119) (width 0.2) (layer "F.Cu") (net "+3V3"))
 (segment (start 133.5 131.19) (end 132.31 130) (width 0.2) (layer "F.Cu") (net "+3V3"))
 (segment (start 86.588 122.169895) (end 86.588 118.334105) (width 0.2) (layer "F.Cu") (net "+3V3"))
 (segment (start 87.65 82.572) (end 87.65 114.11) (width 0.2) (layer "F.Cu") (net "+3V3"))
 (segment (start 86.588 118.334105) (end 87.210105 117.712) (width 0.2) (layer "F.Cu") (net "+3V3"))
 (segment (start 88.712 117.089895) (end 88.712 116.210105) (width 0.2) (layer "F.Cu") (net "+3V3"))
 (segment (start 109.46 134.04) (end 109.46 127.8275) (width 0.2) (layer "F.Cu") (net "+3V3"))
 (segment (start 87.210105 117.712) (end 88.089895 117.712) (width 0.2) (layer "F.Cu") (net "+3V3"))
 (segment (start 89 115.46) (end 89 118) (width 0.2) (layer "F.Cu") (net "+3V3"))
 (segment (start 83.846315 115.588) (end 82.6 116.834315) (width 0.2) (layer "F.Cu") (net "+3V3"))
 (segment (start 112.5 116.5) (end 118.6015 116.5) (width 0.2) (layer "F.Cu") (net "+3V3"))
 (segment (start 88.089895 117.712) (end 88.712 117.089895) (width 0.2) (layer "F.Cu") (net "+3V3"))
 (segment (start 109.46 127.8275) (end 109.46 122.54) (width 0.2) (layer "F.Cu") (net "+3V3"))
 (segment (start 87.65 114.11) (end 89 115.46) (width 0.2) (layer "F.Cu") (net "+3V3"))
 (segment (start 90.23 79.992) (end 87.65 82.572) (width 0.2) (layer "F.Cu") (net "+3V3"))
 (segment (start 120.7215 119.69763) (end 117.62713 122.792) (width 0.2) (layer "F.Cu") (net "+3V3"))
 (segment (start 133.5 137) (end 133.5 131.19) (width 0.2) (layer "F.Cu") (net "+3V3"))
 (segment (start 118.6015 116.5) (end 120.7215 118.62) (width 0.2) (layer "F.Cu") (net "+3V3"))
 (segment (start 112 117) (end 112.5 116.5) (width 0.2) (layer "F.Cu") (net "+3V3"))
 (segment (start 89 118) (end 85 118) (width 0.2) (layer "F.Cu") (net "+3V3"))
 (segment (start 85 134.5) (end 109 134.5) (width 0.2) (layer "F.Cu") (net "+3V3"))
 (segment (start 112 121) (end 112 117) (width 0.2) (layer "F.Cu") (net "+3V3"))
 (segment (start 84 119) (end 84 133.5) (width 0.2) (layer "F.Cu") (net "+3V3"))
 (segment (start 82.6 135.5) (end 84.1 137) (width 0.2) (layer "F.Cu") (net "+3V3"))
 (segment (start 120.7215 118.62) (end 120.7215 119.69763) (width 0.2) (layer "F.Cu") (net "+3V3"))
 (segment (start 87.210105 122.792) (end 86.588 122.169895) (width 0.2) (layer "F.Cu") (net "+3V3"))
 (segment (start 82.6 116.834315) (end 82.6 135.5) (width 0.2) (layer "F.Cu") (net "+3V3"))
 (segment (start 117.62713 122.792) (end 87.210105 122.792) (width 0.2) (layer "F.Cu") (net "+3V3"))
 (segment (start 110 122) (end 111 122) (width 0.2) (layer "F.Cu") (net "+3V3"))
 (segment (start 84.1 137) (end 133.5 137) (width 0.2) (layer "F.Cu") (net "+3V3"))
 (segment (start 109 134.5) (end 109.46 134.04) (width 0.2) (layer "F.Cu") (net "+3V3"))
 (segment (start 88.089895 115.588) (end 83.846315 115.588) (width 0.2) (layer "F.Cu") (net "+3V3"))
 (segment (start 123.2615 103.38) (end 126.8635 106.982) (width 0.2) (layer "F.Cu") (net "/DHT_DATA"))
 (segment (start 114 134.5) (end 124 134.5) (width 0.2) (layer "F.Cu") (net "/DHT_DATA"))
 (segment (start 112 132.5) (end 114 134.5) (width 0.2) (layer "F.Cu") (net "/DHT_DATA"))
 (segment (start 124 134.5) (end 124.69 133.81) (width 0.2) (layer "F.Cu") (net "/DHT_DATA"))
 (segment (start 112 127.8275) (end 112 132.5) (width 0.2) (layer "F.Cu") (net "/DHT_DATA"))
 (segment (start 126.8635 127.8265) (end 124.69 130) (width 0.2) (layer "F.Cu") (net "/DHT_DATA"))
 (segment (start 124.69 133.81) (end 124.69 130) (width 0.2) (layer "F.Cu") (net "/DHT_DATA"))
 (segment (start 126.8635 106.982) (end 126.8635 127.8265) (width 0.2) (layer "F.Cu") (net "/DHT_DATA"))
 (segment (start 83.35 116.65) (end 83 117) (width 0.2) (layer "F.Cu") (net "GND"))
 (segment (start 87.65 116.65) (end 83.35 116.65) (width 0.2) (layer "F.Cu") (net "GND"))
 (segment (start 111.5 123.5) (end 117 123.5) (width 0.2) (layer "F.Cu") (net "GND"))
 (segment (start 118.63 81.52) (end 132.75 81.52) (width 0.2) (layer "F.Cu") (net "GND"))
 (segment (start 107.807 78.577) (end 114.69 85.46) (width 0.2) (layer "F.Cu") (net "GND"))
 (segment (start 110.95 135.45) (end 110.95 124.05) (width 0.2) (layer "F.Cu") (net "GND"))
 (segment (start 117 110.5) (end 119.5 113) (width 0.2) (layer "F.Cu") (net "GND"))
 (segment (start 117 123.5) (end 117.08 123.58) (width 0.2) (layer "F.Cu") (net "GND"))
 (segment (start 117 98.31) (end 117 110.5) (width 0.2) (layer "F.Cu") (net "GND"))
 (segment (start 111 135.5) (end 110.95 135.45) (width 0.2) (layer "F.Cu") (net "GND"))
 (segment (start 83 117) (end 83 135) (width 0.2) (layer "F.Cu") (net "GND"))
 (segment (start 132.75 81.52) (end 136.69 85.46) (width 0.2) (layer "F.Cu") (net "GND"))
 (segment (start 83 135) (end 83.5 135.5) (width 0.2) (layer "F.Cu") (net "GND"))
 (segment (start 114.69 96) (end 117 98.31) (width 0.2) (layer "F.Cu") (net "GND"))
 (segment (start 110.95 124.05) (end 111.5 123.5) (width 0.2) (layer "F.Cu") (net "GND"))
 (segment (start 123.2615 118.62) (end 123.2615 119.69763) (width 0.2) (layer "F.Cu") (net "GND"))
 (segment (start 114.69 85.46) (end 118.63 81.52) (width 0.2) (layer "F.Cu") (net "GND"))
 (segment (start 117.08 123.58) (end 117.08 127.8275) (width 0.2) (layer "F.Cu") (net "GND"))
 (segment (start 114.69 85.46) (end 114.69 96) (width 0.2) (layer "F.Cu") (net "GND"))
 (segment (start 123.2615 119.69763) (end 119.37913 123.58) (width 0.2) (layer "F.Cu") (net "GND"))
 (segment (start 87.69 79.992) (end 89.105 78.577) (width 0.2) (layer "F.Cu") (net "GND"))
 (segment (start 119.5 113) (end 119.5 114.8585) (width 0.2) (layer "F.Cu") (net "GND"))
 (segment (start 119.5 114.8585) (end 123.2615 118.62) (width 0.2) (layer "F.Cu") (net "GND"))
 (segment (start 119.37913 123.58) (end 117.08 123.58) (width 0.2) (layer "F.Cu") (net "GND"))
 (segment (start 83.5 135.5) (end 111 135.5) (width 0.2) (layer "F.Cu") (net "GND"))
 (segment (start 89.105 78.577) (end 107.807 78.577) (width 0.2) (layer "F.Cu") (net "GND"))
 (segment (start 87.65 119.19) (end 88.34 118.5) (width 0.2) (layer "F.Cu") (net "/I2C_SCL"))
 (segment (start 88.34 118.5) (end 90 118.5) (width 0.2) (layer "F.Cu") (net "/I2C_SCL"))
 (segment (start 101.585862 106) (end 102.5 106) (width 0.2) (layer "F.Cu") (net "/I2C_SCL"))
 (segment (start 110.4815 106) (end 113.1015 103.38) (width 0.2) (layer "F.Cu") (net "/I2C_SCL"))
 (segment (start 92.77 97.184138) (end 101.585862 106) (width 0.2) (layer "F.Cu") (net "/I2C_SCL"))
 (segment (start 92.77 79.992) (end 92.77 97.184138) (width 0.2) (layer "F.Cu") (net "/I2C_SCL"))
 (segment (start 102.5 106) (end 110.4815 106) (width 0.2) (layer "F.Cu") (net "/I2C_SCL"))
 (segment (start 90 118.5) (end 102.5 106) (width 0.2) (layer "F.Cu") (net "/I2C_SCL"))
 (segment (start 114.1635 103.819895) (end 110.983395 107) (width 0.2) (layer "F.Cu") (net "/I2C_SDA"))
 (segment (start 105 107) (end 110.983395 107) (width 0.2) (layer "F.Cu") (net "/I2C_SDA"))
 (segment (start 90.27 121.73) (end 105 107) (width 0.2) (layer "F.Cu") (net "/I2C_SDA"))
 (segment (start 114.1635 98.8455) (end 114.1635 103.819895) (width 0.2) (layer "F.Cu") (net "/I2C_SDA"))
 (segment (start 112.5 106.5215) (end 115.6415 103.38) (width 0.2) (layer "F.Cu") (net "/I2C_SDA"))
 (segment (start 110.983395 107) (end 112.5 107) (width 0.2) (layer "F.Cu") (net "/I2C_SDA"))
 (segment (start 95.31 79.992) (end 114.1635 98.8455) (width 0.2) (layer "F.Cu") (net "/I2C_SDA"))
 (segment (start 112.5 107) (end 112.5 106.5215) (width 0.2) (layer "F.Cu") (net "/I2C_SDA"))
 (segment (start 87.65 121.73) (end 90.27 121.73) (width 0.2) (layer "F.Cu") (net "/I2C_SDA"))
 (segment (start 121.04 103.0615) (end 120.7215 103.38) (width 0.2) (layer "F.Cu") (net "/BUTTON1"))
 (segment (start 121.04 82.92) (end 121.04 103.0615) (width 0.2) (layer "F.Cu") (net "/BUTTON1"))
 (segment (start 126.117056 99) (end 142.197056 82.92) (width 0.2) (layer "F.Cu") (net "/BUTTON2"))
 (segment (start 123 99) (end 126.117056 99) (width 0.2) (layer "F.Cu") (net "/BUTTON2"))
 (segment (start 121.3015 106.5) (end 122 106.5) (width 0.2) (layer "F.Cu") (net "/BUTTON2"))
 (segment (start 122 106.5) (end 122 100) (width 0.2) (layer "F.Cu") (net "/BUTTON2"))
 (segment (start 122 100) (end 123 99) (width 0.2) (layer "F.Cu") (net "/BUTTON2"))
 (segment (start 118.1815 103.38) (end 121.3015 106.5) (width 0.2) (layer "F.Cu") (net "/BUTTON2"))
 (segment (start 142.197056 82.92) (end 143.04 82.92) (width 0.2) (layer "F.Cu") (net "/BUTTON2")))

